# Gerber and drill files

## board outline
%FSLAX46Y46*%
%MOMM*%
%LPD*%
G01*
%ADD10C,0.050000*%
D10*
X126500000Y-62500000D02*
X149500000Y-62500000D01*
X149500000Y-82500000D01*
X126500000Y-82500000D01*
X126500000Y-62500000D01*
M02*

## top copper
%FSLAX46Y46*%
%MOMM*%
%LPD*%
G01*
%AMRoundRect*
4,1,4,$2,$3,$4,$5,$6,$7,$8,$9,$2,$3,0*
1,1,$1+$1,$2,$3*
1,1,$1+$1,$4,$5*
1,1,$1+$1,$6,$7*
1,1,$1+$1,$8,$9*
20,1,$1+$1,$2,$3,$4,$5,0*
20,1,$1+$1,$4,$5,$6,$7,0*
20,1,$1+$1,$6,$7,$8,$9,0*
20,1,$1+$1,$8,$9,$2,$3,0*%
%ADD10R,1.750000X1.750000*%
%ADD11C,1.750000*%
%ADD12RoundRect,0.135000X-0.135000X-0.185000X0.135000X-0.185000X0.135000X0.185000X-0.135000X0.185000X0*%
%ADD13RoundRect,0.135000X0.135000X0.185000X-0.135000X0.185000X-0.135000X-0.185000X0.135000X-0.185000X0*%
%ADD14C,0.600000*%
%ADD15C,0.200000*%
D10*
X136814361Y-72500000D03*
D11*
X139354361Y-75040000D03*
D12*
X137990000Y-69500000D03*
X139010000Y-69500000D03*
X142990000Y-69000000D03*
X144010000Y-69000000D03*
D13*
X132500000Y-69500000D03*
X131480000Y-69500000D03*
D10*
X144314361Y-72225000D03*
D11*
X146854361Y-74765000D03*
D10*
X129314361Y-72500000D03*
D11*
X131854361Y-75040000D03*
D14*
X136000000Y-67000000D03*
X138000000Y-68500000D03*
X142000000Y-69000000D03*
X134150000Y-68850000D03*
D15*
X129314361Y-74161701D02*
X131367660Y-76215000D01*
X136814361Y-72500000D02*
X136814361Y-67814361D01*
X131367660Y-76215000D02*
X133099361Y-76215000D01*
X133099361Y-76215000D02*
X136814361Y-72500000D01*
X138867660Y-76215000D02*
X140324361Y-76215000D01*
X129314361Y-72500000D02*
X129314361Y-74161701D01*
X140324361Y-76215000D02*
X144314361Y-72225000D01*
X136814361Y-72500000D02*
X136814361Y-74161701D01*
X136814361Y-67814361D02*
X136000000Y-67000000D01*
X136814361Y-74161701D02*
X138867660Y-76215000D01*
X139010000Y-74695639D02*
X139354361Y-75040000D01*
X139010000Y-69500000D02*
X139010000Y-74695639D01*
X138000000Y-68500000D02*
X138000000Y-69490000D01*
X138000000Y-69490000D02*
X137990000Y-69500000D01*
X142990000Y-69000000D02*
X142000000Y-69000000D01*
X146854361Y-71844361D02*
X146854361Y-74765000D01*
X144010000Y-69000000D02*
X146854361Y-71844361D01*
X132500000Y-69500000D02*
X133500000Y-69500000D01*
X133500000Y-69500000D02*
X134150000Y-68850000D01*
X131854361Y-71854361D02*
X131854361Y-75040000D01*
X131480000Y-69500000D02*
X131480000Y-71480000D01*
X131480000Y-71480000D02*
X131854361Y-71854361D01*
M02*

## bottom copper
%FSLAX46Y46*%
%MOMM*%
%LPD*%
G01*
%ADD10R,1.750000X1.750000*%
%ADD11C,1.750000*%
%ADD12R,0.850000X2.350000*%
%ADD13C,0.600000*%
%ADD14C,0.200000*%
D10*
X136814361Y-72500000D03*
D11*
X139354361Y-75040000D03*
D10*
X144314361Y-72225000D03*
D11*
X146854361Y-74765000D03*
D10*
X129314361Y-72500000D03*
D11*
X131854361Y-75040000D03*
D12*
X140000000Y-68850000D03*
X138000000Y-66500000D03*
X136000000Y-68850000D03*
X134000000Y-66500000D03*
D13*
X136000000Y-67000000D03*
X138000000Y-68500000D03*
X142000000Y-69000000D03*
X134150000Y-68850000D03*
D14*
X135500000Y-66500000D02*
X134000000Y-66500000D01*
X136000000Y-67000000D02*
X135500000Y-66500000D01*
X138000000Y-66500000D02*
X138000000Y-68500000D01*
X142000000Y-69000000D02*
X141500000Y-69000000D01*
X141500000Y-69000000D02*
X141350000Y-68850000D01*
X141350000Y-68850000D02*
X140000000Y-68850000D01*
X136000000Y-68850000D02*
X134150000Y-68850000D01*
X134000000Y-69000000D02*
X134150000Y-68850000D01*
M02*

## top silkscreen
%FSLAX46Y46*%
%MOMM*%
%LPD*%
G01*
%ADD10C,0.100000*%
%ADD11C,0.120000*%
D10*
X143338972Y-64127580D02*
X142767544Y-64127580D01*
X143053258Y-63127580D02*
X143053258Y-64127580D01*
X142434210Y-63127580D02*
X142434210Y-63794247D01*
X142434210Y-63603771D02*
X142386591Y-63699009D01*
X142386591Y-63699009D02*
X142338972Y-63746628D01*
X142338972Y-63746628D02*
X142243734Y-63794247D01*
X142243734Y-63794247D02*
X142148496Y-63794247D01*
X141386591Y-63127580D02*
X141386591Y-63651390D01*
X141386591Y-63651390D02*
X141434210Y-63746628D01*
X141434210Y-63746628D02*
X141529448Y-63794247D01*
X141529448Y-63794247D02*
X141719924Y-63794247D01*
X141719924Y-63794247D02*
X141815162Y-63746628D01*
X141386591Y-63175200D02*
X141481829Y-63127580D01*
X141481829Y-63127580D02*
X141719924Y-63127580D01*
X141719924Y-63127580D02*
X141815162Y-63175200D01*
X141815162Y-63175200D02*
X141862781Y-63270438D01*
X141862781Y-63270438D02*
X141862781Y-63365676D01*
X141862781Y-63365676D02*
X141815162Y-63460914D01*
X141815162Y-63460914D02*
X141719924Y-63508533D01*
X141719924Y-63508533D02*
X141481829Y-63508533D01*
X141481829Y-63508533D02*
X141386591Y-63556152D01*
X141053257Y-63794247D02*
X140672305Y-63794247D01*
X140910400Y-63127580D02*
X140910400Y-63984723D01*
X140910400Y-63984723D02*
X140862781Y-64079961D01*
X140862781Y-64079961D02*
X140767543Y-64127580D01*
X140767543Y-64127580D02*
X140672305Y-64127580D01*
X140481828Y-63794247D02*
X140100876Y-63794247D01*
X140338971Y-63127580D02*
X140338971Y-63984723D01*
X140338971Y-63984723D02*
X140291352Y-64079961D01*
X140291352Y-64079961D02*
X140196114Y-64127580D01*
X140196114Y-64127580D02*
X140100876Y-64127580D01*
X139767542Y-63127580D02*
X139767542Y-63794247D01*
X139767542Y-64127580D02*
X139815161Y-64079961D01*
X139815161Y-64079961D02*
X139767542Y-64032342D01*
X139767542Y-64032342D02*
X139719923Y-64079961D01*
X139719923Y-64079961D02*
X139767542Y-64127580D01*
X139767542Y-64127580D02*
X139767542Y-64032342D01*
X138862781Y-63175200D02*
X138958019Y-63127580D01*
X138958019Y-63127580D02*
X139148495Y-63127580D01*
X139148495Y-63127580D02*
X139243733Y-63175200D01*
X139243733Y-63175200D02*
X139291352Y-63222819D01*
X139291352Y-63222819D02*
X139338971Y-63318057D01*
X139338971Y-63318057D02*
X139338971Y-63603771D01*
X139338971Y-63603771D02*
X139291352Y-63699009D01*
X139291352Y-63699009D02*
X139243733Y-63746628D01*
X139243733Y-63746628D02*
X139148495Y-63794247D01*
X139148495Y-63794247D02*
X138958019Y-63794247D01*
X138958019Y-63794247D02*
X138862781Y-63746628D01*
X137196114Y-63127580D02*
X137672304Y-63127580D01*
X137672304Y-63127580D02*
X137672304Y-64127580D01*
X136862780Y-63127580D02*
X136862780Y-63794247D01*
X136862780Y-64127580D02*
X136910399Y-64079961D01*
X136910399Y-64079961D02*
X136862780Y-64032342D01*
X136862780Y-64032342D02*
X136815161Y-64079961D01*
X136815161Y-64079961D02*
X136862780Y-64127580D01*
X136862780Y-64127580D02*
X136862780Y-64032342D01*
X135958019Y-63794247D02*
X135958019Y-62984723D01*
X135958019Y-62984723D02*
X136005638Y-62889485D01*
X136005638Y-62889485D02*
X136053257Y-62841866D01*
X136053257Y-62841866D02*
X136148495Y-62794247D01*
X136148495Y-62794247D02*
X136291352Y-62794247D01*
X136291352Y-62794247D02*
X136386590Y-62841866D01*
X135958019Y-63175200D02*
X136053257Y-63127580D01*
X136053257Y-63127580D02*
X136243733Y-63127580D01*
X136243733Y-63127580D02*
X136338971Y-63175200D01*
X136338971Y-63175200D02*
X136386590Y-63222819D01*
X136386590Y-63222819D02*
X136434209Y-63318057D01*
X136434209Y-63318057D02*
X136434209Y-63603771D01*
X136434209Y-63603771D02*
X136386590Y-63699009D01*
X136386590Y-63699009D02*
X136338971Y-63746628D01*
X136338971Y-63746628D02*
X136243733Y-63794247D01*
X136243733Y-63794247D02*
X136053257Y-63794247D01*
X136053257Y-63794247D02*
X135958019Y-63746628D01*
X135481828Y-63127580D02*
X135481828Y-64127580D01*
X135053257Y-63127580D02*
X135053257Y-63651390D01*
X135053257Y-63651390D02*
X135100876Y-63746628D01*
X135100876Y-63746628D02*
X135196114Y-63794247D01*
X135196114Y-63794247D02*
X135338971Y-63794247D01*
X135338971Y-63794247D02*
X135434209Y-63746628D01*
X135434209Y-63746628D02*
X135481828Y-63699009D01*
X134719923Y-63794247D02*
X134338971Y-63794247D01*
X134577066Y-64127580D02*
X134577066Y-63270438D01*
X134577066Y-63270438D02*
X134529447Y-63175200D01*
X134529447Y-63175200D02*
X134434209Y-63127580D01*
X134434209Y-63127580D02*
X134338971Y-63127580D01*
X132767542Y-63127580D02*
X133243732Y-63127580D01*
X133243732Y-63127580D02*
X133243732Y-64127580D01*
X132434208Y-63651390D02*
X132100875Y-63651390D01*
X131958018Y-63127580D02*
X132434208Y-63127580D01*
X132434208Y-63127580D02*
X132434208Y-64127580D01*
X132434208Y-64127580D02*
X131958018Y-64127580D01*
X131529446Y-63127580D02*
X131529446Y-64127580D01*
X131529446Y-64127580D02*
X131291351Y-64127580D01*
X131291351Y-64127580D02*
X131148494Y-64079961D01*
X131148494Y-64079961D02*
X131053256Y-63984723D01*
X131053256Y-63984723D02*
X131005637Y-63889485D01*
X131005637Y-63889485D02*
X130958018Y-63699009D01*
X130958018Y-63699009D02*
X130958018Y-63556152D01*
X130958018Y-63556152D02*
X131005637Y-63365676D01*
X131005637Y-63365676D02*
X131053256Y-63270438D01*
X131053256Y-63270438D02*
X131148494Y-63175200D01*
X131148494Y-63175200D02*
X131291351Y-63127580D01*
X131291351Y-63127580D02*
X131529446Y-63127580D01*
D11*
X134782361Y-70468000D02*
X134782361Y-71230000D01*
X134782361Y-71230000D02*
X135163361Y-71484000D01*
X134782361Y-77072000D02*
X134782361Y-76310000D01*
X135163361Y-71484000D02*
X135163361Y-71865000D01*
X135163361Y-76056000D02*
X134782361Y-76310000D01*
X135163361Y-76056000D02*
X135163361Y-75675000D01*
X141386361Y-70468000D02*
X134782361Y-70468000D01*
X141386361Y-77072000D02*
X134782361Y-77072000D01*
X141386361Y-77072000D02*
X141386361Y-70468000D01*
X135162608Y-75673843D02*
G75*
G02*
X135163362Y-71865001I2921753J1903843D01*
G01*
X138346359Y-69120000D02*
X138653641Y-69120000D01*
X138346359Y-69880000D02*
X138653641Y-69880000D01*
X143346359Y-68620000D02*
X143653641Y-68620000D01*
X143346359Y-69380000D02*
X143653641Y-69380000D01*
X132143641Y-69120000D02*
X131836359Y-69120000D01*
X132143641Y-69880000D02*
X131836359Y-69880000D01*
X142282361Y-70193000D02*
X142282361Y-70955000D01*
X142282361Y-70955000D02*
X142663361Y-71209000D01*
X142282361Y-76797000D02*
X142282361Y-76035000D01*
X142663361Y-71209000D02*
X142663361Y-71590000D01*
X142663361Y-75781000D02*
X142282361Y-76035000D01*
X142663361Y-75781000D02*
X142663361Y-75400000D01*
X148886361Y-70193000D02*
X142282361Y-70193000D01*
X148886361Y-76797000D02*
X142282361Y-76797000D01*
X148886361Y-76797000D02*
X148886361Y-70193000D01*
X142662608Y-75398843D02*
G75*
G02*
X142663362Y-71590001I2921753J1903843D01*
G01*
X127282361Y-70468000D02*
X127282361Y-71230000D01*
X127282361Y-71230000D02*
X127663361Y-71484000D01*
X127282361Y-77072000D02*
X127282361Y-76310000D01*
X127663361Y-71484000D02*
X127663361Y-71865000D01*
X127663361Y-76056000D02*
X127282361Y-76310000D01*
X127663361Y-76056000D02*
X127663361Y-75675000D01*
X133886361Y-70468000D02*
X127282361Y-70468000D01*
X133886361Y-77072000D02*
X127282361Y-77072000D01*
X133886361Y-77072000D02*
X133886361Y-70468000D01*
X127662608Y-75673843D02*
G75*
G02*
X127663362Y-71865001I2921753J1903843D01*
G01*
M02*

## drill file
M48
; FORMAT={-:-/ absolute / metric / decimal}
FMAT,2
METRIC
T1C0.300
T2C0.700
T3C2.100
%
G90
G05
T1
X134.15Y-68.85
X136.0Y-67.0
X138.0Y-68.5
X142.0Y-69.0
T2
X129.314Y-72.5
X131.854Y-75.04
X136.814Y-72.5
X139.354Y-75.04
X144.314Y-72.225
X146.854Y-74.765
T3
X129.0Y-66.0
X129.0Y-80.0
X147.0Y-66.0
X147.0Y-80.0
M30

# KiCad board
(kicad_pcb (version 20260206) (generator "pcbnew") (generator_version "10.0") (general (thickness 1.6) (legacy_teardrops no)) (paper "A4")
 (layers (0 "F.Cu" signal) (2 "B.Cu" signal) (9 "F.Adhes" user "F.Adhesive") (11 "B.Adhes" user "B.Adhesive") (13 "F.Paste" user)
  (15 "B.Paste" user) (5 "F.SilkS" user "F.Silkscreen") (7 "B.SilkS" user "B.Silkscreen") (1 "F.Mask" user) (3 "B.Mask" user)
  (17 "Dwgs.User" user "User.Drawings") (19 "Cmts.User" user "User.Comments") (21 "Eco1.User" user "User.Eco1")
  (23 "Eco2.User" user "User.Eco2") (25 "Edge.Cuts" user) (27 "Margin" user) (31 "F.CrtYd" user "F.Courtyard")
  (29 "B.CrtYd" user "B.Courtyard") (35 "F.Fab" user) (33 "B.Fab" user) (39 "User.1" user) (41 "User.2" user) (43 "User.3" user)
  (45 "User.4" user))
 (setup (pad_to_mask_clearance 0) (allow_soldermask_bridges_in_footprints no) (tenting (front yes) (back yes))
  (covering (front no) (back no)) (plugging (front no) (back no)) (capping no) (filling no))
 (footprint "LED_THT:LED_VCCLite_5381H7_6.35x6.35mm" (layer "F.Cu") (at 136.814361 72.5)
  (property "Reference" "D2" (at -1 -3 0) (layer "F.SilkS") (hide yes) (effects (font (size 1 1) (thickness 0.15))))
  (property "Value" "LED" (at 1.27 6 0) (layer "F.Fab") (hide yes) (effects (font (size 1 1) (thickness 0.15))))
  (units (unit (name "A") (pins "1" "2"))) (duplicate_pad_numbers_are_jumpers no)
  (fp_line (start -2.032 -2.032) (end -2.032 -1.27) (stroke (width 0.12) (type solid)) (layer "F.SilkS"))
  (fp_line (start -2.032 -1.27) (end -1.651 -1.016) (stroke (width 0.12) (type solid)) (layer "F.SilkS"))
  (fp_line (start -2.032 4.572) (end -2.032 3.81) (stroke (width 0.12) (type solid)) (layer "F.SilkS"))
  (fp_line (start -1.651 -1.016) (end -1.651 -0.635) (stroke (width 0.12) (type solid)) (layer "F.SilkS"))
  (fp_line (start -1.651 3.556) (end -2.032 3.81) (stroke (width 0.12) (type solid)) (layer "F.SilkS"))
  (fp_line (start -1.651 3.556) (end -1.651 3.175) (stroke (width 0.12) (type solid)) (layer "F.SilkS"))
  (fp_line (start 4.572 -2.032) (end -2.032 -2.032) (stroke (width 0.12) (type solid)) (layer "F.SilkS"))
  (fp_line (start 4.572 4.572) (end -2.032 4.572) (stroke (width 0.12) (type solid)) (layer "F.SilkS"))
  (fp_line (start 4.572 4.572) (end 4.572 -2.032) (stroke (width 0.12) (type solid)) (layer "F.SilkS"))
  (fp_arc (start -1.651753 3.173843) (mid -2.2173 1.26931) (end -1.650999 -0.634999) (stroke (width 0.12) (type solid)) (layer "F.SilkS"))
  (pad "1" thru_hole rect (at 0 0 270) (size 1.75 1.75) (drill 0.7) (layers "*.Cu" "*.Mask") (remove_unused_layers no) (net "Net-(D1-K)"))
  (pad "2" thru_hole circle (at 2.54 2.54 270) (size 1.75 1.75) (drill 0.7) (layers "*.Cu" "*.Mask") (remove_unused_layers no)
   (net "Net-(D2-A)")))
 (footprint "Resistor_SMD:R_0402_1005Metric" (layer "F.Cu") (at 138.5 69.5)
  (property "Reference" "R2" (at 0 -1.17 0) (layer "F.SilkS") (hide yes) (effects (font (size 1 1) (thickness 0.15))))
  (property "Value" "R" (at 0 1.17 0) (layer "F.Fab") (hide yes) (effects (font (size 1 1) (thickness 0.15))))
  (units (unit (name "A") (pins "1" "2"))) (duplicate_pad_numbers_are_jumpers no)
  (fp_line (start -0.153641 -0.38) (end 0.153641 -0.38) (stroke (width 0.12) (type solid)) (layer "F.SilkS"))
  (fp_line (start -0.153641 0.38) (end 0.153641 0.38) (stroke (width 0.12) (type solid)) (layer "F.SilkS"))
  (pad "1" smd roundrect (at -0.51 0) (size 0.54 0.64) (layers "F.Cu" "F.Mask" "F.Paste") (roundrect_rratio 0.25) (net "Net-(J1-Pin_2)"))
  (pad "2" smd roundrect (at 0.51 0) (size 0.54 0.64) (layers "F.Cu" "F.Mask" "F.Paste") (roundrect_rratio 0.25) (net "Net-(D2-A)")))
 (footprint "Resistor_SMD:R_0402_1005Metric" (layer "F.Cu") (at 143.5 69)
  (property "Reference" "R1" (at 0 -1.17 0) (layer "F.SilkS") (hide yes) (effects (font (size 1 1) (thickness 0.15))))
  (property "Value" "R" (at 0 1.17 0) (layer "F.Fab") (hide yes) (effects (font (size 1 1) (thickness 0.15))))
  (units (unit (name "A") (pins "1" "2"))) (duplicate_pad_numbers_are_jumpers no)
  (fp_line (start -0.153641 -0.38) (end 0.153641 -0.38) (stroke (width 0.12) (type solid)) (layer "F.SilkS"))
  (fp_line (start -0.153641 0.38) (end 0.153641 0.38) (stroke (width 0.12) (type solid)) (layer "F.SilkS"))
  (pad "1" smd roundrect (at -0.51 0) (size 0.54 0.64) (layers "F.Cu" "F.Mask" "F.Paste") (roundrect_rratio 0.25) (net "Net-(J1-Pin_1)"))
  (pad "2" smd roundrect (at 0.51 0) (size 0.54 0.64) (layers "F.Cu" "F.Mask" "F.Paste") (roundrect_rratio 0.25) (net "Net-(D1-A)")))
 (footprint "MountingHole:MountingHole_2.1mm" (layer "F.Cu") (at 147 80)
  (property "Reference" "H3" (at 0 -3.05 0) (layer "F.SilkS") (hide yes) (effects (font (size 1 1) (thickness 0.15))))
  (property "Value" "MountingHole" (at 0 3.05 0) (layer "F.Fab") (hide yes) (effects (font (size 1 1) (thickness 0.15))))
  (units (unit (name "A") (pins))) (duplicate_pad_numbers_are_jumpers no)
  (pad "" np_thru_hole circle (at 0 0) (size 2.1 2.1) (drill 2.1) (layers "*.Cu" "*.Mask")))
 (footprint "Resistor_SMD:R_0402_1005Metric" (layer "F.Cu") (at 131.99 69.5 180)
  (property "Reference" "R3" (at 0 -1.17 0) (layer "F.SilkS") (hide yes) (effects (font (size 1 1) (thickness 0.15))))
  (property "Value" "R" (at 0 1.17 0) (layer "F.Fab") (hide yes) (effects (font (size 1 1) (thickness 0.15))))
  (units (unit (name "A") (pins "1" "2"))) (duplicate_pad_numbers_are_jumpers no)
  (fp_line (start -0.153641 0.38) (end 0.153641 0.38) (stroke (width 0.12) (type solid)) (layer "F.SilkS"))
  (fp_line (start -0.153641 -0.38) (end 0.153641 -0.38) (stroke (width 0.12) (type solid)) (layer "F.SilkS"))
  (pad "1" smd roundrect (at -0.51 0 180) (size 0.54 0.64) (layers "F.Cu" "F.Mask" "F.Paste") (roundrect_rratio 0.25) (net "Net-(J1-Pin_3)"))
  (pad "2" smd roundrect (at 0.51 0 180) (size 0.54 0.64) (layers "F.Cu" "F.Mask" "F.Paste") (roundrect_rratio 0.25) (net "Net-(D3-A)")))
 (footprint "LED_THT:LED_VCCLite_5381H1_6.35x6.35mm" (layer "F.Cu") (at 144.314361 72.225)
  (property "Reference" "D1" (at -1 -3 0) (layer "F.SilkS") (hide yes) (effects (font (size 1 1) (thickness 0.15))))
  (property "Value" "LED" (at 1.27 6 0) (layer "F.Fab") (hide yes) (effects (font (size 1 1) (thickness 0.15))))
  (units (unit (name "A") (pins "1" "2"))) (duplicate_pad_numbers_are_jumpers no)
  (fp_line (start -2.032 -2.032) (end -2.032 -1.27) (stroke (width 0.12) (type solid)) (layer "F.SilkS"))
  (fp_line (start -2.032 -1.27) (end -1.651 -1.016) (stroke (width 0.12) (type solid)) (layer "F.SilkS"))
  (fp_line (start -2.032 4.572) (end -2.032 3.81) (stroke (width 0.12) (type solid)) (layer "F.SilkS"))
  (fp_line (start -1.651 -1.016) (end -1.651 -0.635) (stroke (width 0.12) (type solid)) (layer "F.SilkS"))
  (fp_line (start -1.651 3.556) (end -2.032 3.81) (stroke (width 0.12) (type solid)) (layer "F.SilkS"))
  (fp_line (start -1.651 3.556) (end -1.651 3.175) (stroke (width 0.12) (type solid)) (layer "F.SilkS"))
  (fp_line (start 4.572 -2.032) (end -2.032 -2.032) (stroke (width 0.12) (type solid)) (layer "F.SilkS"))
  (fp_line (start 4.572 4.572) (end -2.032 4.572) (stroke (width 0.12) (type solid)) (layer "F.SilkS"))
  (fp_line (start 4.572 4.572) (end 4.572 -2.032) (stroke (width 0.12) (type solid)) (layer "F.SilkS"))
  (fp_arc (start -1.651753 3.173843) (mid -2.2173 1.26931) (end -1.650999 -0.634999) (stroke (width 0.12) (type solid)) (layer "F.SilkS"))
  (pad "1" thru_hole rect (at 0 0 270) (size 1.75 1.75) (drill 0.7) (layers "*.Cu" "*.Mask") (remove_unused_layers no) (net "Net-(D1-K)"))
  (pad "2" thru_hole circle (at 2.54 2.54 270) (size 1.75 1.75) (drill 0.7) (layers "*.Cu" "*.Mask") (remove_unused_layers no)
   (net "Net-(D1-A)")))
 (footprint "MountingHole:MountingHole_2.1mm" (layer "F.Cu") (at 129 80)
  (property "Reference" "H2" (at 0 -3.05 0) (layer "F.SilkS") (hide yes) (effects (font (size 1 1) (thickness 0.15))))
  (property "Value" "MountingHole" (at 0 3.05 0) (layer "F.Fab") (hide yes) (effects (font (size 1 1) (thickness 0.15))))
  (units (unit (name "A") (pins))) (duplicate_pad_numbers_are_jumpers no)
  (pad "" np_thru_hole circle (at 0 0) (size 2.1 2.1) (drill 2.1) (layers "*.Cu" "*.Mask")))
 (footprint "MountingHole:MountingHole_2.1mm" (layer "F.Cu") (at 129 66)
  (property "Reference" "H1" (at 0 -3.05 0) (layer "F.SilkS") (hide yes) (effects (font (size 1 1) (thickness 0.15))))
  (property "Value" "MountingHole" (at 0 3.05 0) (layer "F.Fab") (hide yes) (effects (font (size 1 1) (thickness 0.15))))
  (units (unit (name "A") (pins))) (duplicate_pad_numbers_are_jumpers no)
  (pad "" np_thru_hole circle (at 0 0) (size 2.1 2.1) (drill 2.1) (layers "*.Cu" "*.Mask")))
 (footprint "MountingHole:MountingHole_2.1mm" (layer "F.Cu") (at 147 66)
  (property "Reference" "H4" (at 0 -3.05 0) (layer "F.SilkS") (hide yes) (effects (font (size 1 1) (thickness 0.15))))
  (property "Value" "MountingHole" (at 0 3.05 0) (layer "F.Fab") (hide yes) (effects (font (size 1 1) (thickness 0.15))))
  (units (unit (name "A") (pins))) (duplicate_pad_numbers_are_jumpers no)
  (pad "" np_thru_hole circle (at 0 0) (size 2.1 2.1) (drill 2.1) (layers "*.Cu" "*.Mask")))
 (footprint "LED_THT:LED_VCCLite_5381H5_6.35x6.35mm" (layer "F.Cu") (at 129.314361 72.5)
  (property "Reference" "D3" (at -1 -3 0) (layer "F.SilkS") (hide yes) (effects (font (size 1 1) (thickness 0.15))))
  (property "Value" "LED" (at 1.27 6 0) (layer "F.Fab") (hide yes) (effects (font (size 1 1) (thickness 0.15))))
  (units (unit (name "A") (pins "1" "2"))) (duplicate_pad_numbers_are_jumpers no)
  (fp_line (start -2.032 -2.032) (end -2.032 -1.27) (stroke (width 0.12) (type solid)) (layer "F.SilkS"))
  (fp_line (start -2.032 -1.27) (end -1.651 -1.016) (stroke (width 0.12) (type solid)) (layer "F.SilkS"))
  (fp_line (start -2.032 4.572) (end -2.032 3.81) (stroke (width 0.12) (type solid)) (layer "F.SilkS"))
  (fp_line (start -1.651 -1.016) (end -1.651 -0.635) (stroke (width 0.12) (type solid)) (layer "F.SilkS"))
  (fp_line (start -1.651 3.556) (end -2.032 3.81) (stroke (width 0.12) (type solid)) (layer "F.SilkS"))
  (fp_line (start -1.651 3.556) (end -1.651 3.175) (stroke (width 0.12) (type solid)) (layer "F.SilkS"))
  (fp_line (start 4.572 -2.032) (end -2.032 -2.032) (stroke (width 0.12) (type solid)) (layer "F.SilkS"))
  (fp_line (start 4.572 4.572) (end -2.032 4.572) (stroke (width 0.12) (type solid)) (layer "F.SilkS"))
  (fp_line (start 4.572 4.572) (end 4.572 -2.032) (stroke (width 0.12) (type solid)) (layer "F.SilkS"))
  (fp_arc (start -1.651753 3.173843) (mid -2.2173 1.26931) (end -1.650999 -0.634999) (stroke (width 0.12) (type solid)) (layer "F.SilkS"))
  (pad "1" thru_hole rect (at 0 0 270) (size 1.75 1.75) (drill 0.7) (layers "*.Cu" "*.Mask") (remove_unused_layers no) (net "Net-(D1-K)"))
  (pad "2" thru_hole circle (at 2.54 2.54 270) (size 1.75 1.75) (drill 0.7) (layers "*.Cu" "*.Mask") (remove_unused_layers no)
   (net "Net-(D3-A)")))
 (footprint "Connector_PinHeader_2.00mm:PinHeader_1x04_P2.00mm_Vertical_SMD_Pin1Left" (layer "B.Cu") (at 137 67.675 90)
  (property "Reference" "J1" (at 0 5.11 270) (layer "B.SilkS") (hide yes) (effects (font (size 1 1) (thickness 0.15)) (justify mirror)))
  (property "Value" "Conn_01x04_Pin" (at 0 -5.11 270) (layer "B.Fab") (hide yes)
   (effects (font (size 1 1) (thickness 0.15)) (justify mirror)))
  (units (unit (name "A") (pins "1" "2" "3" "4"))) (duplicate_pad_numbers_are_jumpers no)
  (pad "1" smd rect (at -1.175 3 90) (size 2.35 0.85) (layers "B.Cu" "B.Mask" "B.Paste") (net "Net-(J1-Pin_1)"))
  (pad "2" smd rect (at 1.175 1 90) (size 2.35 0.85) (layers "B.Cu" "B.Mask" "B.Paste") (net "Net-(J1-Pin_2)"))
  (pad "3" smd rect (at -1.175 -1 90) (size 2.35 0.85) (layers "B.Cu" "B.Mask" "B.Paste") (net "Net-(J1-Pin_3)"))
  (pad "4" smd rect (at 1.175 -3 90) (size 2.35 0.85) (layers "B.Cu" "B.Mask" "B.Paste") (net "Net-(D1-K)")))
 (gr_rect (start 126.5 62.5) (end 149.5 82.5) (stroke (width 0.05) (type default)) (fill no) (layer "Edge.Cuts"))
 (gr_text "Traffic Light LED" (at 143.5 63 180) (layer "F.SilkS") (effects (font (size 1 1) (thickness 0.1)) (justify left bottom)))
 (segment (start 129.314361 74.161701) (end 131.36766 76.215) (width 0.2) (layer "F.Cu") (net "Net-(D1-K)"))
 (segment (start 136.814361 72.5) (end 136.814361 67.814361) (width 0.2) (layer "F.Cu") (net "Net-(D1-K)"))
 (segment (start 131.36766 76.215) (end 133.099361 76.215) (width 0.2) (layer "F.Cu") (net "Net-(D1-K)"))
 (segment (start 133.099361 76.215) (end 136.814361 72.5) (width 0.2) (layer "F.Cu") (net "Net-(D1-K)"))
 (segment (start 138.86766 76.215) (end 140.324361 76.215) (width 0.2) (layer "F.Cu") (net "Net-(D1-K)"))
 (segment (start 129.314361 72.5) (end 129.314361 74.161701) (width 0.2) (layer "F.Cu") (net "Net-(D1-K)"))
 (segment (start 140.324361 76.215) (end 144.314361 72.225) (width 0.2) (layer "F.Cu") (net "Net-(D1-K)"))
 (segment (start 136.814361 72.5) (end 136.814361 74.161701) (width 0.2) (layer "F.Cu") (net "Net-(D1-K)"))
 (segment (start 136.814361 67.814361) (end 136 67) (width 0.2) (layer "F.Cu") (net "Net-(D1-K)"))
 (segment (start 136.814361 74.161701) (end 138.86766 76.215) (width 0.2) (layer "F.Cu") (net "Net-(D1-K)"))
 (via (at 136 67) (size 0.6) (drill 0.3) (layers "F.Cu" "B.Cu") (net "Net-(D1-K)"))
 (segment (start 135.5 66.5) (end 134 66.5) (width 0.2) (layer "B.Cu") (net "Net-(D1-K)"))
 (segment (start 136 67) (end 135.5 66.5) (width 0.2) (layer "B.Cu") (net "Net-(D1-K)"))
 (segment (start 139.01 74.695639) (end 139.354361 75.04) (width 0.2) (layer "F.Cu") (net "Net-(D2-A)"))
 (segment (start 139.01 69.5) (end 139.01 74.695639) (width 0.2) (layer "F.Cu") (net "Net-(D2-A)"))
 (segment (start 138 68.5) (end 138 69.49) (width 0.2) (layer "F.Cu") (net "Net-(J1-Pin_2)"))
 (segment (start 138 69.49) (end 137.99 69.5) (width 0.2) (layer "F.Cu") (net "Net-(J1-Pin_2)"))
 (via (at 138 68.5) (size 0.6) (drill 0.3) (layers "F.Cu" "B.Cu") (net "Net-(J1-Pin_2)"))
 (segment (start 138 66.5) (end 138 68.5) (width 0.2) (layer "B.Cu") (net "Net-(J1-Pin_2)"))
 (segment (start 142.99 69) (end 142 69) (width 0.2) (layer "F.Cu") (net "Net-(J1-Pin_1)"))
 (via (at 142 69) (size 0.6) (drill 0.3) (layers "F.Cu" "B.Cu") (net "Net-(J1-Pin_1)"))
 (segment (start 142 69) (end 141.5 69) (width 0.2) (layer "B.Cu") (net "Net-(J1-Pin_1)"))
 (segment (start 141.5 69) (end 141.35 68.85) (width 0.2) (layer "B.Cu") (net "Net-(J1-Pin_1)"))
 (segment (start 141.35 68.85) (end 140 68.85) (width 0.2) (layer "B.Cu") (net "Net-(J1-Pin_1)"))
 (segment (start 146.854361 71.844361) (end 146.854361 74.765) (width 0.2) (layer "F.Cu") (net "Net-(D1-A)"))
 (segment (start 144.01 69) (end 146.854361 71.844361) (width 0.2) (layer "F.Cu") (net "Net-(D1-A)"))
 (segment (start 132.5 69.5) (end 133.5 69.5) (width 0.2) (layer "F.Cu") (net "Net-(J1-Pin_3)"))
 (segment (start 133.5 69.5) (end 134.15 68.85) (width 0.2) (layer "F.Cu") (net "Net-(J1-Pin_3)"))
 (via (at 134.15 68.85) (size 0.6) (drill 0.3) (layers "F.Cu" "B.Cu") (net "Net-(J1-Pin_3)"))
 (segment (start 136 68.85) (end 134.15 68.85) (width 0.2) (layer "B.Cu") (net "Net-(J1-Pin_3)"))
 (segment (start 134 69) (end 134.15 68.85) (width 0.2) (layer "B.Cu") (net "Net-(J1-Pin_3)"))
 (segment (start 131.854361 71.854361) (end 131.854361 75.04) (width 0.2) (layer "F.Cu") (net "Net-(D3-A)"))
 (segment (start 131.48 69.5) (end 131.48 71.48) (width 0.2) (layer "F.Cu") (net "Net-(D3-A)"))
 (segment (start 131.48 71.48) (end 131.854361 71.854361) (width 0.2) (layer "F.Cu") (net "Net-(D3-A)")))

